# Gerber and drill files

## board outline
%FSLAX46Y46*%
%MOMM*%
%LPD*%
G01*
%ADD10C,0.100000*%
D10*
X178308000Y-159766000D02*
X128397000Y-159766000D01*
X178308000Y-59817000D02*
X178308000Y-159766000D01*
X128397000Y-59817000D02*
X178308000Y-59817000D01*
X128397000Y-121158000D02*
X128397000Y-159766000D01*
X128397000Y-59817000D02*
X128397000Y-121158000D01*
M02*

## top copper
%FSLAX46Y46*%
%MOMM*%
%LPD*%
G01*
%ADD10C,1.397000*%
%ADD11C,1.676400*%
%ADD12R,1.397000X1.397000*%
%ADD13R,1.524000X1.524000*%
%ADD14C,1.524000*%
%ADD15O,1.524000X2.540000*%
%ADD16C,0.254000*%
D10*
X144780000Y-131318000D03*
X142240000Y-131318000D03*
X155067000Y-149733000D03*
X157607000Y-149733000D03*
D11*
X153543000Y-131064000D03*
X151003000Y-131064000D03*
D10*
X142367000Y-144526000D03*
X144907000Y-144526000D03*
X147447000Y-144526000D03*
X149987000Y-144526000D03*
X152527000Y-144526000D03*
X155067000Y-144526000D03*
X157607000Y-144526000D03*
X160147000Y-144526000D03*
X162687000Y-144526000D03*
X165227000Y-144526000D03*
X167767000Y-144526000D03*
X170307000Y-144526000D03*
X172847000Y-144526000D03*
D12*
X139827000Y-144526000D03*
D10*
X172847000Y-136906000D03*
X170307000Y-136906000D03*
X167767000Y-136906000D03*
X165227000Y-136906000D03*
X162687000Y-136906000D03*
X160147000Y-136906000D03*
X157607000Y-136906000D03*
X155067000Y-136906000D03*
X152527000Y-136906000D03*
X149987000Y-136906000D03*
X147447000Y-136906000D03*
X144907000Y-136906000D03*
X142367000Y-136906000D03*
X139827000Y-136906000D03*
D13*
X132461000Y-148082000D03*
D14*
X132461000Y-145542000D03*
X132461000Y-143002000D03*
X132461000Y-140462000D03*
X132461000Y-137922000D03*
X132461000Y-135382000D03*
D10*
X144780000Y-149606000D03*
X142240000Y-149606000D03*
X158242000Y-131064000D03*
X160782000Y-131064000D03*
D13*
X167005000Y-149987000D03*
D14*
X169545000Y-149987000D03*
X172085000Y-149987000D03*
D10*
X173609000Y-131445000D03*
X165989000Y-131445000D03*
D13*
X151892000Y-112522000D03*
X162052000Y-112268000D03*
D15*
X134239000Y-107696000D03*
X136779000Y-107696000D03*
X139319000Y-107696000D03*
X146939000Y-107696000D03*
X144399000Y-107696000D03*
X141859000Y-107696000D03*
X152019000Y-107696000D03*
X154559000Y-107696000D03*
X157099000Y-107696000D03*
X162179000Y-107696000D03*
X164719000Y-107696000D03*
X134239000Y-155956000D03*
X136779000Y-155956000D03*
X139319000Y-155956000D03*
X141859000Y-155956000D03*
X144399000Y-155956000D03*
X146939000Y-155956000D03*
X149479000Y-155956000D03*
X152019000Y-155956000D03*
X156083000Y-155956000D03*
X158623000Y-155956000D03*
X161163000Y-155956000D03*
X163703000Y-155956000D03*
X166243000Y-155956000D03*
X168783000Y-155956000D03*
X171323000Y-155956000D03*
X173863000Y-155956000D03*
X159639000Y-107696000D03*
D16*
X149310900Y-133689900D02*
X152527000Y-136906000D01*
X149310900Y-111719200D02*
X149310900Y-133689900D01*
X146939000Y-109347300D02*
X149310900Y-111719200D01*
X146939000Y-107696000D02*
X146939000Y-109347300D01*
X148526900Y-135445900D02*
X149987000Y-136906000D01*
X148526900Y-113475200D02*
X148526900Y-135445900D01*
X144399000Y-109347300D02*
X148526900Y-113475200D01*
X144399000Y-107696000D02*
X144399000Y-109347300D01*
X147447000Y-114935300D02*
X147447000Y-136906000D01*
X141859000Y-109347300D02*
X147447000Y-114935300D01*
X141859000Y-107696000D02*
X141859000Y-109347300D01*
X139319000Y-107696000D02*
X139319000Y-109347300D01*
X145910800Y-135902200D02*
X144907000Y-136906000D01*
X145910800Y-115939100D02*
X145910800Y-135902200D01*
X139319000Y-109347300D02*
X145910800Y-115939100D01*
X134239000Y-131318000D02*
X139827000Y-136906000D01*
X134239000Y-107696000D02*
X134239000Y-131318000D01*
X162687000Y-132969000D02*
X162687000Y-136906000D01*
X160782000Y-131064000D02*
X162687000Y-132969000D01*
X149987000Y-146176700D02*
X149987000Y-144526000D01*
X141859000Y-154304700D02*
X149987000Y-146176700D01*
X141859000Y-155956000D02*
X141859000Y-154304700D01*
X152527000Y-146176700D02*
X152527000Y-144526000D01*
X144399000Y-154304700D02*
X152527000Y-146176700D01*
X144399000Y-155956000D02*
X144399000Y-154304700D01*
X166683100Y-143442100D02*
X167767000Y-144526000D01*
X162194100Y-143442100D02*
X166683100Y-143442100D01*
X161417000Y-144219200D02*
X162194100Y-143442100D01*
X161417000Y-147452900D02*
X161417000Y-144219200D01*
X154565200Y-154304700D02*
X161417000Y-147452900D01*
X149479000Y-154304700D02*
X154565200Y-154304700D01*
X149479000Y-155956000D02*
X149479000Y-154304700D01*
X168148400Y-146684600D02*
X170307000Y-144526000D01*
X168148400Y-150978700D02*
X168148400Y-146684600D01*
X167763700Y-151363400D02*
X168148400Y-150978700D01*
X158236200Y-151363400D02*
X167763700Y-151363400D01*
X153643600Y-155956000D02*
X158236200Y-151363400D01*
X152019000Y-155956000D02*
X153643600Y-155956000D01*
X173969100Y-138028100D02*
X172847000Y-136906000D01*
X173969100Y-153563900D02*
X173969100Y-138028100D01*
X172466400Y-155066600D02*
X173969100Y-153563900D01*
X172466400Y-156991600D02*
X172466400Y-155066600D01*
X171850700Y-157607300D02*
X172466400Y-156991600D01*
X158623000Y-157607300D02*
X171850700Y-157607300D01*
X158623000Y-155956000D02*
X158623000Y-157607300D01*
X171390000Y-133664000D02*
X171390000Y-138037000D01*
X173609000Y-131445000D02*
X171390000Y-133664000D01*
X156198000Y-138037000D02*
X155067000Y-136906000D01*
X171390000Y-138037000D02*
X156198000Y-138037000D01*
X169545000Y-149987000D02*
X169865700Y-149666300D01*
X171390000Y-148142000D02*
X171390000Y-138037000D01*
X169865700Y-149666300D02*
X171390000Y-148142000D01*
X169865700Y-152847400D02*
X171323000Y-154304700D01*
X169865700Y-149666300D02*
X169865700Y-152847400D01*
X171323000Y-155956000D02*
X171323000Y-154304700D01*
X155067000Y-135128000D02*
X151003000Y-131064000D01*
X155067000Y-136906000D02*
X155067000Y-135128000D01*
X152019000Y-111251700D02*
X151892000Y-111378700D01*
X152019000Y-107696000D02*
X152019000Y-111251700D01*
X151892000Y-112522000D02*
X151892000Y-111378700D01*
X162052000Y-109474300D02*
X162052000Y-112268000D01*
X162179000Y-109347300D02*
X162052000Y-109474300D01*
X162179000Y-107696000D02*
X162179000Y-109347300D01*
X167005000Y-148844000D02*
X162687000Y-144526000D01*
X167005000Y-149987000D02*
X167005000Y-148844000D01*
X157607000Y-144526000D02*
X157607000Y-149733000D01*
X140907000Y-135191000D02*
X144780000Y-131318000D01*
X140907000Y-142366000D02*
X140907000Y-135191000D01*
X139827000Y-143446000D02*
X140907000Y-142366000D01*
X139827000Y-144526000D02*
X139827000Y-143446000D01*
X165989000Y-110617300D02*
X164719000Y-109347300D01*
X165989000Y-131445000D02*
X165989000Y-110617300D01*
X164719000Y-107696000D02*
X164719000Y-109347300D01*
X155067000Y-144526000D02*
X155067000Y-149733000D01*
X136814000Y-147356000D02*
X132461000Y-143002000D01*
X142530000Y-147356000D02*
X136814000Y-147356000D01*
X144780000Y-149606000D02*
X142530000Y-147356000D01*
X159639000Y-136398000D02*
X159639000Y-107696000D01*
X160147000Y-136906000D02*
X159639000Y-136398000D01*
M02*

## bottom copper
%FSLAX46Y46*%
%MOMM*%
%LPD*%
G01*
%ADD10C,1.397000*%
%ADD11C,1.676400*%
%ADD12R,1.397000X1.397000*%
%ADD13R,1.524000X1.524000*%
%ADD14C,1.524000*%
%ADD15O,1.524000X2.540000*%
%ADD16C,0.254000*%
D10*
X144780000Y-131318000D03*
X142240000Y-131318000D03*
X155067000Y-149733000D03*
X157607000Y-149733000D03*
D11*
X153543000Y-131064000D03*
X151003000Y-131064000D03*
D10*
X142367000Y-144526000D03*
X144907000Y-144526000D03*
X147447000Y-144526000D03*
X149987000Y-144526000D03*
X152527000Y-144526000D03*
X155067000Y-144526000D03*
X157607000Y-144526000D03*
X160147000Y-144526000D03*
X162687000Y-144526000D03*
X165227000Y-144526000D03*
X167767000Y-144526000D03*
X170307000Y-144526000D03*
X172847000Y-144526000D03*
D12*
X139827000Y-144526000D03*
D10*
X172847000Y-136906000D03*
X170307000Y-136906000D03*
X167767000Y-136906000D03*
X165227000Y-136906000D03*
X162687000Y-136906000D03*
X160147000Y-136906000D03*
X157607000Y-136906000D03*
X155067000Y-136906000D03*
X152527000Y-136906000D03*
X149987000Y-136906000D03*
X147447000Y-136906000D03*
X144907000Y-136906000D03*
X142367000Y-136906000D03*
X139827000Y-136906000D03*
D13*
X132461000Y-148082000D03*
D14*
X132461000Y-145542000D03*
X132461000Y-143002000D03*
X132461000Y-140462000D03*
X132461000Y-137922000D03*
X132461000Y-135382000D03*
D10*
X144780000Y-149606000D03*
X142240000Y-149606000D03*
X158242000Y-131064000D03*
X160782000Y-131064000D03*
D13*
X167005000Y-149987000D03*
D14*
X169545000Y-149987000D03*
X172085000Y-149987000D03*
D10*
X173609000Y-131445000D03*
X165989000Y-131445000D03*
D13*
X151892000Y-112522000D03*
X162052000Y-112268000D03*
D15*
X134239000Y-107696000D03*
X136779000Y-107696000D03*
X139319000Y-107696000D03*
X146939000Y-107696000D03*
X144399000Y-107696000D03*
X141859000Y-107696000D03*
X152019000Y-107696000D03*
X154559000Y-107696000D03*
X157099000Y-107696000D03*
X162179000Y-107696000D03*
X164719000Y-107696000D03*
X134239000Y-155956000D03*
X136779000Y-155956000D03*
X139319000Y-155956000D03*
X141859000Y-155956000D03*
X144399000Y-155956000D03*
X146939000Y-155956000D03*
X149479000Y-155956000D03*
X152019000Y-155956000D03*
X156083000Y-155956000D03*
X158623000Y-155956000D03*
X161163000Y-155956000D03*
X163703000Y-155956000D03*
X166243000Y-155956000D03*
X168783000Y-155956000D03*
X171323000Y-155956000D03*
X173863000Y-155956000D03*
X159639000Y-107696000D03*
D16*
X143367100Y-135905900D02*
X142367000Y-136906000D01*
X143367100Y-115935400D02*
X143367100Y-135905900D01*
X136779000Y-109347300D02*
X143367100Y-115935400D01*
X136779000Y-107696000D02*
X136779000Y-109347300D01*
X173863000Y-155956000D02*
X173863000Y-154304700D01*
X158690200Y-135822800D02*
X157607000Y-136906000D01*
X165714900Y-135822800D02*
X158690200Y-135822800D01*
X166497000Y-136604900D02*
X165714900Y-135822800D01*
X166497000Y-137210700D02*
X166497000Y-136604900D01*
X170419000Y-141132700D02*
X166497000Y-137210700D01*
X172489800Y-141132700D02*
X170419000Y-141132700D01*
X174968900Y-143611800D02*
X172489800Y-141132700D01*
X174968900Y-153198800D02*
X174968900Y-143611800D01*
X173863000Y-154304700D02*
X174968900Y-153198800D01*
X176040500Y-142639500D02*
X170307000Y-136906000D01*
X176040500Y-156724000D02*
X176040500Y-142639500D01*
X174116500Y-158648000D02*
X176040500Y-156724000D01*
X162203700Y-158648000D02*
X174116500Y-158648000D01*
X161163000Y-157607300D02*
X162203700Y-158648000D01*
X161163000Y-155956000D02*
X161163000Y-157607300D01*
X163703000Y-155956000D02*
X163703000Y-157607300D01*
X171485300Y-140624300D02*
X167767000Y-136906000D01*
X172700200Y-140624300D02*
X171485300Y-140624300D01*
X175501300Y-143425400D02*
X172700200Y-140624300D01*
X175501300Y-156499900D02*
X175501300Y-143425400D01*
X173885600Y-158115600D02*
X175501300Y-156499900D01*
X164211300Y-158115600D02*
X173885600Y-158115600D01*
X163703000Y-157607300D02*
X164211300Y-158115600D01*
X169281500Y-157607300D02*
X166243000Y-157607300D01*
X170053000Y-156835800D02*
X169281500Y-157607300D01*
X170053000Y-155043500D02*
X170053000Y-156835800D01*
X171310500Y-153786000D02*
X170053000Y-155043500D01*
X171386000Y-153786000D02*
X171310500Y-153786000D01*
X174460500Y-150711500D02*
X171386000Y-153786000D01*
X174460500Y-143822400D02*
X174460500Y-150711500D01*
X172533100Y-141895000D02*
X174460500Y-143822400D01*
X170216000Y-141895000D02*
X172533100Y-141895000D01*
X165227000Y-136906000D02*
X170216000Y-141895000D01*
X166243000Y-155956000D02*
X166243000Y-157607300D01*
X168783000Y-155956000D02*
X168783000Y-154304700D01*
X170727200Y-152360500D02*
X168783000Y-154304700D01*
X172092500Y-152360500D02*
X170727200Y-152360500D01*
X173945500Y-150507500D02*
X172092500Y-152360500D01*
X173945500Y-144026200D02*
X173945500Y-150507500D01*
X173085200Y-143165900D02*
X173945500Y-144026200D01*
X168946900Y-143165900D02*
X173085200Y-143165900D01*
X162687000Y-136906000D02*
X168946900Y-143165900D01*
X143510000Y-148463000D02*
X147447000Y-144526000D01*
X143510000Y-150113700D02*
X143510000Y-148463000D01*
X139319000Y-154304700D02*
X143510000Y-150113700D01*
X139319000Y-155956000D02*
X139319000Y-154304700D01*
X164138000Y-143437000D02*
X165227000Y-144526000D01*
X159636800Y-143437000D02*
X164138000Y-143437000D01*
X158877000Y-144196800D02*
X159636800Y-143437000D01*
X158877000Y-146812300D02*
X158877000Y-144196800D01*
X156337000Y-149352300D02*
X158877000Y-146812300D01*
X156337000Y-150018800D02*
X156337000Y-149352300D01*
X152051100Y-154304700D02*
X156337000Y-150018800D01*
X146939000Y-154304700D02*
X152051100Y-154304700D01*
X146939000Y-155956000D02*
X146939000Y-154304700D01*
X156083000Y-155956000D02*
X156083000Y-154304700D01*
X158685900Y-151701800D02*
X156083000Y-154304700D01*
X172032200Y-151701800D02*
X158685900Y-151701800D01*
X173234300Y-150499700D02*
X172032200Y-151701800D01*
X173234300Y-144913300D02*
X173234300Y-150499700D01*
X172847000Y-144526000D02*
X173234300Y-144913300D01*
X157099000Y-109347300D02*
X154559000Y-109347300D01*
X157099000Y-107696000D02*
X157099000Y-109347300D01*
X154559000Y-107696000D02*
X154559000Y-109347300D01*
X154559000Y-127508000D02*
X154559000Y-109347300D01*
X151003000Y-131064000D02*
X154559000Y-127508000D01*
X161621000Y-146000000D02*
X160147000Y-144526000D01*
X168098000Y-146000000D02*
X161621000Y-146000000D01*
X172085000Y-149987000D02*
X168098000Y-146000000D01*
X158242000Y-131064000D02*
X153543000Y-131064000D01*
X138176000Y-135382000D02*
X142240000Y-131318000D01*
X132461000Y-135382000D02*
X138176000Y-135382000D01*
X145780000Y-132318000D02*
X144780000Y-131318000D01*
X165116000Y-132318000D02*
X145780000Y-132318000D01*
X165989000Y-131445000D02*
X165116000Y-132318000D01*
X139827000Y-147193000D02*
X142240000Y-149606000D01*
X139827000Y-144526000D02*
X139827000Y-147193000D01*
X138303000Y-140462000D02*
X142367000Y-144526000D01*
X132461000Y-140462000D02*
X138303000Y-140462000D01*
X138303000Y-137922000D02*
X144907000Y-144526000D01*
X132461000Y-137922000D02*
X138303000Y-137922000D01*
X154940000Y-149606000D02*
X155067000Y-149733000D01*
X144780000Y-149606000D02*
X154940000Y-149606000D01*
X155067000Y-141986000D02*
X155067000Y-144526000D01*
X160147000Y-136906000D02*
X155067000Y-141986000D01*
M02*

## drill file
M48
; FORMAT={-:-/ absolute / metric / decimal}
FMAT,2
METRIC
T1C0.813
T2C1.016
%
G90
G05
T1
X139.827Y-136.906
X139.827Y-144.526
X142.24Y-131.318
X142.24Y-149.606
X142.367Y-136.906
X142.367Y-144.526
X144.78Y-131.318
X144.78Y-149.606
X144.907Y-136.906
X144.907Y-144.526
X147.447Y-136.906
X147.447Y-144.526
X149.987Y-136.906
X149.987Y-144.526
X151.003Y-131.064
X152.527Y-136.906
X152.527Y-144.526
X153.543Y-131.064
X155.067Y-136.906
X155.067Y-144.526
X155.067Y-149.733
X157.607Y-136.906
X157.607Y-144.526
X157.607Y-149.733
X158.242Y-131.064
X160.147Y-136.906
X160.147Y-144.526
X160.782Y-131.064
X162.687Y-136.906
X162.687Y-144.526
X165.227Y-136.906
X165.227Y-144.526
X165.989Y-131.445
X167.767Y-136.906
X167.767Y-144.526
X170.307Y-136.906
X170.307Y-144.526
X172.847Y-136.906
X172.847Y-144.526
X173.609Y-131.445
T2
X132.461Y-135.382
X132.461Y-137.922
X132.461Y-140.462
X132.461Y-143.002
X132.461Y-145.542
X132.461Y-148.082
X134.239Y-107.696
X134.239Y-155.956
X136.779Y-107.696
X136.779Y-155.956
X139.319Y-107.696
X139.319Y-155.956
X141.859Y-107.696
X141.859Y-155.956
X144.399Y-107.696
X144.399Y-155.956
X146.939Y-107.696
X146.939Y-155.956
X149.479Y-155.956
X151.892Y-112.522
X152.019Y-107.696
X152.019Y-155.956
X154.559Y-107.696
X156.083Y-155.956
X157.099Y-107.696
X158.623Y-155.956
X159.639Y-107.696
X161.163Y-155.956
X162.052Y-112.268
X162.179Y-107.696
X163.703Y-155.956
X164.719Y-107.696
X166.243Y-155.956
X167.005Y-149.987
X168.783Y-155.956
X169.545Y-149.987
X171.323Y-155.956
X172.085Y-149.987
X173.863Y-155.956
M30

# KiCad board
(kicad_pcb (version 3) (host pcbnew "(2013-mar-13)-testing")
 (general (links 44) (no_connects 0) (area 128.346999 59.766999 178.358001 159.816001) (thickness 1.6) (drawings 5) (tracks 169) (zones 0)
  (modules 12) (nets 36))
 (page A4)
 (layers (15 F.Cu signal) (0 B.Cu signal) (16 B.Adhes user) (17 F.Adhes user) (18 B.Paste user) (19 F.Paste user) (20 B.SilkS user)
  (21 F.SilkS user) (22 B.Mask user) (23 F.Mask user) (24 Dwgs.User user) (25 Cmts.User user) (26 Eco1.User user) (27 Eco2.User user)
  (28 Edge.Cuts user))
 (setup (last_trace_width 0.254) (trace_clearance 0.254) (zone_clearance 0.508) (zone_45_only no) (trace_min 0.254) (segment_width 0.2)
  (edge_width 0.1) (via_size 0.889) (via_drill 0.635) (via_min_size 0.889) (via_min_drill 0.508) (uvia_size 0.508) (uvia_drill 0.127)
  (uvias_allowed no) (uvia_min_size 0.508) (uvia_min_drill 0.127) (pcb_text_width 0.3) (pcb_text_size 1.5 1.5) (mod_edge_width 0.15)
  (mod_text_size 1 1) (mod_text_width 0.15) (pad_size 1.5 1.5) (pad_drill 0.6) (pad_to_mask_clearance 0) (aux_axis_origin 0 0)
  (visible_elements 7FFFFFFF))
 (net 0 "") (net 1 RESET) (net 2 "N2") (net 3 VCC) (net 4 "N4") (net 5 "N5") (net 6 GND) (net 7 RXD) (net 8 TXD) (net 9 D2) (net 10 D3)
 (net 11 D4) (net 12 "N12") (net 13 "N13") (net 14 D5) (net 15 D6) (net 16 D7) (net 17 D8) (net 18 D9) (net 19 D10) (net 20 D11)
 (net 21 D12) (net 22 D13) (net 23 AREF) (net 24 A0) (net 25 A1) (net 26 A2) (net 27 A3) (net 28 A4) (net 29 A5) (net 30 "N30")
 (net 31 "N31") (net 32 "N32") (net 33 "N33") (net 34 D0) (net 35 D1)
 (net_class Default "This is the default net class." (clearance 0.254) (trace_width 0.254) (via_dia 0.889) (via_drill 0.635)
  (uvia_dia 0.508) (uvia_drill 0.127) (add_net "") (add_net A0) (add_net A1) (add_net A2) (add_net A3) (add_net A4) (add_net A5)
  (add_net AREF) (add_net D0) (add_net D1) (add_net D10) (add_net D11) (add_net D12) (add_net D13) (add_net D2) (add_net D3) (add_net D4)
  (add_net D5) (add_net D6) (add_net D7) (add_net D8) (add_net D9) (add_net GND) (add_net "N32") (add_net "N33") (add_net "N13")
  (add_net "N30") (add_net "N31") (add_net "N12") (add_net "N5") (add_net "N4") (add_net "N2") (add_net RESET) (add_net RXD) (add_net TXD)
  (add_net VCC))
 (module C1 (layer F.Cu) (at 143.51 131.318 180)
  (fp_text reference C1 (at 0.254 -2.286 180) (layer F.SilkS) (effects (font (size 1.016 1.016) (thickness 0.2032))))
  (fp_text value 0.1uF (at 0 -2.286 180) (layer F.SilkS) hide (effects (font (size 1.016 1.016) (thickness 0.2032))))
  (pad 1 thru_hole circle (at -1.27 0 180) (size 1.397 1.397) (drill 0.8128) (layers *.Cu *.Mask F.SilkS) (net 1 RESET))
  (pad 2 thru_hole circle (at 1.27 0 180) (size 1.397 1.397) (drill 0.8128) (layers *.Cu *.Mask F.SilkS) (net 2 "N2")))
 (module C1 (layer F.Cu) (at 156.337 149.733)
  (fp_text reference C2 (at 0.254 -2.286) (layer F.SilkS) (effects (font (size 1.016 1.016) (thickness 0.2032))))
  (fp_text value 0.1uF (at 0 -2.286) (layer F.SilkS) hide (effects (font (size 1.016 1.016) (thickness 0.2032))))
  (pad 1 thru_hole circle (at -1.27 0) (size 1.397 1.397) (drill 0.8128) (layers *.Cu *.Mask F.SilkS) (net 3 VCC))
  (pad 2 thru_hole circle (at 1.27 0) (size 1.397 1.397) (drill 0.8128) (layers *.Cu *.Mask F.SilkS) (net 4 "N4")))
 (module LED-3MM (layer F.Cu) (at 152.273 131.064 180)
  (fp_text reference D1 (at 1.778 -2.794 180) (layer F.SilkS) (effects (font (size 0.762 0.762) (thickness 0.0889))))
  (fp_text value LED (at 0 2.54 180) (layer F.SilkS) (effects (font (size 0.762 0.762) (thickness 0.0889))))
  (pad 1 thru_hole circle (at -1.27 0 180) (size 1.6764 1.6764) (drill 0.8128) (layers *.Cu *.Mask F.SilkS) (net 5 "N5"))
  (pad 2 thru_hole circle (at 1.27 0 180) (size 1.6764 1.6764) (drill 0.8128) (layers *.Cu *.Mask F.SilkS) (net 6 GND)))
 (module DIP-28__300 (layer F.Cu) (at 156.337 140.716)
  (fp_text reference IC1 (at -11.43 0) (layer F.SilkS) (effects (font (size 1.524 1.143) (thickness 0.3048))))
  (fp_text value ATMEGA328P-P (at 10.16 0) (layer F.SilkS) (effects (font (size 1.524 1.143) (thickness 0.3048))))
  (pad 2 thru_hole circle (at -13.97 3.81) (size 1.397 1.397) (drill 0.8128) (layers *.Cu *.Mask F.SilkS) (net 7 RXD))
  (pad 3 thru_hole circle (at -11.43 3.81) (size 1.397 1.397) (drill 0.8128) (layers *.Cu *.Mask F.SilkS) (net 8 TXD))
  (pad 4 thru_hole circle (at -8.89 3.81) (size 1.397 1.397) (drill 0.8128) (layers *.Cu *.Mask F.SilkS) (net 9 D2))
  (pad 5 thru_hole circle (at -6.35 3.81) (size 1.397 1.397) (drill 0.8128) (layers *.Cu *.Mask F.SilkS) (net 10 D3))
  (pad 6 thru_hole circle (at -3.81 3.81) (size 1.397 1.397) (drill 0.8128) (layers *.Cu *.Mask F.SilkS) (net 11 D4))
  (pad 7 thru_hole circle (at -1.27 3.81) (size 1.397 1.397) (drill 0.8128) (layers *.Cu *.Mask F.SilkS) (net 3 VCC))
  (pad 8 thru_hole circle (at 1.27 3.81) (size 1.397 1.397) (drill 0.8128) (layers *.Cu *.Mask F.SilkS) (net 4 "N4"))
  (pad 9 thru_hole circle (at 3.81 3.81) (size 1.397 1.397) (drill 0.8128) (layers *.Cu *.Mask F.SilkS) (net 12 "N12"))
  (pad 10 thru_hole circle (at 6.35 3.81) (size 1.397 1.397) (drill 0.8128) (layers *.Cu *.Mask F.SilkS) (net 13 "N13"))
  (pad 11 thru_hole circle (at 8.89 3.81) (size 1.397 1.397) (drill 0.8128) (layers *.Cu *.Mask F.SilkS) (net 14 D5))
  (pad 12 thru_hole circle (at 11.43 3.81) (size 1.397 1.397) (drill 0.8128) (layers *.Cu *.Mask F.SilkS) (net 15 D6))
  (pad 13 thru_hole circle (at 13.97 3.81) (size 1.397 1.397) (drill 0.8128) (layers *.Cu *.Mask F.SilkS) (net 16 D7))
  (pad 14 thru_hole circle (at 16.51 3.81) (size 1.397 1.397) (drill 0.8128) (layers *.Cu *.Mask F.SilkS) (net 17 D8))
  (pad 1 thru_hole rect (at -16.51 3.81) (size 1.397 1.397) (drill 0.8128) (layers *.Cu *.Mask F.SilkS) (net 1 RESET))
  (pad 15 thru_hole circle (at 16.51 -3.81) (size 1.397 1.397) (drill 0.8128) (layers *.Cu *.Mask F.SilkS) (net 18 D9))
  (pad 16 thru_hole circle (at 13.97 -3.81) (size 1.397 1.397) (drill 0.8128) (layers *.Cu *.Mask F.SilkS) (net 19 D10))
  (pad 17 thru_hole circle (at 11.43 -3.81) (size 1.397 1.397) (drill 0.8128) (layers *.Cu *.Mask F.SilkS) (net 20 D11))
  (pad 18 thru_hole circle (at 8.89 -3.81) (size 1.397 1.397) (drill 0.8128) (layers *.Cu *.Mask F.SilkS) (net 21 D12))
  (pad 19 thru_hole circle (at 6.35 -3.81) (size 1.397 1.397) (drill 0.8128) (layers *.Cu *.Mask F.SilkS) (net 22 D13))
  (pad 20 thru_hole circle (at 3.81 -3.81) (size 1.397 1.397) (drill 0.8128) (layers *.Cu *.Mask F.SilkS) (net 3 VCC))
  (pad 21 thru_hole circle (at 1.27 -3.81) (size 1.397 1.397) (drill 0.8128) (layers *.Cu *.Mask F.SilkS) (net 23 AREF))
  (pad 22 thru_hole circle (at -1.27 -3.81) (size 1.397 1.397) (drill 0.8128) (layers *.Cu *.Mask F.SilkS) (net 6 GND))
  (pad 23 thru_hole circle (at -3.81 -3.81) (size 1.397 1.397) (drill 0.8128) (layers *.Cu *.Mask F.SilkS) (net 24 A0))
  (pad 24 thru_hole circle (at -6.35 -3.81) (size 1.397 1.397) (drill 0.8128) (layers *.Cu *.Mask F.SilkS) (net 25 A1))
  (pad 25 thru_hole circle (at -8.89 -3.81) (size 1.397 1.397) (drill 0.8128) (layers *.Cu *.Mask F.SilkS) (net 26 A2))
  (pad 26 thru_hole circle (at -11.43 -3.81) (size 1.397 1.397) (drill 0.8128) (layers *.Cu *.Mask F.SilkS) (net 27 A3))
  (pad 27 thru_hole circle (at -13.97 -3.81) (size 1.397 1.397) (drill 0.8128) (layers *.Cu *.Mask F.SilkS) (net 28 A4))
  (pad 28 thru_hole circle (at -16.51 -3.81) (size 1.397 1.397) (drill 0.8128) (layers *.Cu *.Mask F.SilkS) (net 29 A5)))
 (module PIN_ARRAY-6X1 (layer F.Cu) (at 132.461 141.732 90)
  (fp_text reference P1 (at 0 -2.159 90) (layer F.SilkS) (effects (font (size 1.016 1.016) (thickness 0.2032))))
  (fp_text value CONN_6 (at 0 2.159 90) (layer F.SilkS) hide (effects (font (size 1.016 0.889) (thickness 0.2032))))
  (pad 1 thru_hole rect (at -6.35 0 90) (size 1.524 1.524) (drill 1.016) (layers *.Cu *.Mask F.SilkS) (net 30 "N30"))
  (pad 2 thru_hole circle (at -3.81 0 90) (size 1.524 1.524) (drill 1.016) (layers *.Cu *.Mask F.SilkS) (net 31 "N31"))
  (pad 3 thru_hole circle (at -1.27 0 90) (size 1.524 1.524) (drill 1.016) (layers *.Cu *.Mask F.SilkS) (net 3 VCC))
  (pad 4 thru_hole circle (at 1.27 0 90) (size 1.524 1.524) (drill 1.016) (layers *.Cu *.Mask F.SilkS) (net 7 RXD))
  (pad 5 thru_hole circle (at 3.81 0 90) (size 1.524 1.524) (drill 1.016) (layers *.Cu *.Mask F.SilkS) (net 8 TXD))
  (pad 6 thru_hole circle (at 6.35 0 90) (size 1.524 1.524) (drill 1.016) (layers *.Cu *.Mask F.SilkS) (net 2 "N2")))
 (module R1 (layer F.Cu) (at 143.51 149.606 180) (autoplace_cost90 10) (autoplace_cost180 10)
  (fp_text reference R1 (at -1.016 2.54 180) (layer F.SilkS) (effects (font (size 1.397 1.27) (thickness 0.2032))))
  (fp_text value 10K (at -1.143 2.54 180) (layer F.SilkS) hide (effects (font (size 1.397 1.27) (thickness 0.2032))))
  (pad 1 thru_hole circle (at -1.27 0 180) (size 1.397 1.397) (drill 0.8128) (layers *.Cu *.Mask F.SilkS) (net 3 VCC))
  (pad 2 thru_hole circle (at 1.27 0 180) (size 1.397 1.397) (drill 0.8128) (layers *.Cu *.Mask F.SilkS) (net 1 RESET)))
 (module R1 (layer F.Cu) (at 159.512 131.064) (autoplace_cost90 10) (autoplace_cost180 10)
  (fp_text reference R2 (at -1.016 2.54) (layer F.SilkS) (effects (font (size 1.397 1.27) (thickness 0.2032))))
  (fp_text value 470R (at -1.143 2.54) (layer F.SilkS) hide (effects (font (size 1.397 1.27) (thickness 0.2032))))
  (pad 1 thru_hole circle (at -1.27 0) (size 1.397 1.397) (drill 0.8128) (layers *.Cu *.Mask F.SilkS) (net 5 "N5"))
  (pad 2 thru_hole circle (at 1.27 0) (size 1.397 1.397) (drill 0.8128) (layers *.Cu *.Mask F.SilkS) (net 22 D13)))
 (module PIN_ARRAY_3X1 (layer F.Cu) (at 169.545 149.987)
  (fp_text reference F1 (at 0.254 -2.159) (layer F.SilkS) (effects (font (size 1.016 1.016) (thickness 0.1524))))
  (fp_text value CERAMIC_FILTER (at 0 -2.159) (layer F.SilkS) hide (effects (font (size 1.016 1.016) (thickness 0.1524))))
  (pad 1 thru_hole rect (at -2.54 0) (size 1.524 1.524) (drill 1.016) (layers *.Cu *.Mask F.SilkS) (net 13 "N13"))
  (pad 2 thru_hole circle (at 0 0) (size 1.524 1.524) (drill 1.016) (layers *.Cu *.Mask F.SilkS) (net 6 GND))
  (pad 3 thru_hole circle (at 2.54 0) (size 1.524 1.524) (drill 1.016) (layers *.Cu *.Mask F.SilkS) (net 12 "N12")))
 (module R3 (layer F.Cu) (at 169.799 131.445 180) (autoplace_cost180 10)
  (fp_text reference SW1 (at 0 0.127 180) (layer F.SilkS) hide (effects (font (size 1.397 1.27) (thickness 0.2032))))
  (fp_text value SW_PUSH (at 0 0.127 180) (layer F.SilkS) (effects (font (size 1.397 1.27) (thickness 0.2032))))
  (pad 1 thru_hole circle (at -3.81 0 180) (size 1.397 1.397) (drill 0.8128) (layers *.Cu *.Mask F.SilkS) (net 6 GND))
  (pad 2 thru_hole circle (at 3.81 0 180) (size 1.397 1.397) (drill 0.8128) (layers *.Cu *.Mask F.SilkS) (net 1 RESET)))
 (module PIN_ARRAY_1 (layer F.Cu) (at 151.892 112.522)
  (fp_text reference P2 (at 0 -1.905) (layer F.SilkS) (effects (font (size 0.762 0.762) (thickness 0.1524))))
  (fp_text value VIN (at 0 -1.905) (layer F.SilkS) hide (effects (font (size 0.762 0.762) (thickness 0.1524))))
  (pad 1 thru_hole rect (at 0 0) (size 1.524 1.524) (drill 1.016) (layers *.Cu *.Mask F.SilkS) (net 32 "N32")))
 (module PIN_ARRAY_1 (layer F.Cu) (at 162.052 112.268)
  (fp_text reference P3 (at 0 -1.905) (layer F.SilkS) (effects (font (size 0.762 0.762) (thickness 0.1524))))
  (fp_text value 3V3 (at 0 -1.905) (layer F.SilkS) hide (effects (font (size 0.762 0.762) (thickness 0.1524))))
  (pad 1 thru_hole rect (at 0 0) (size 1.524 1.524) (drill 1.016) (layers *.Cu *.Mask F.SilkS) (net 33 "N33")))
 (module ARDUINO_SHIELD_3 (layer F.Cu) (at 174.879 106.426 180)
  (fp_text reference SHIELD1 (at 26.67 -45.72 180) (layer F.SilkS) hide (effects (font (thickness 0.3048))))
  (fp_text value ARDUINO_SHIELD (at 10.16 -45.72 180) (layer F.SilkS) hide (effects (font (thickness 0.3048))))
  (pad AD5 thru_hole oval (at 40.64 -1.27 270) (size 2.54 1.524) (drill 1.016) (layers *.Cu *.Mask F.SilkS) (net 29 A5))
  (pad AD4 thru_hole oval (at 38.1 -1.27 270) (size 2.54 1.524) (drill 1.016) (layers *.Cu *.Mask F.SilkS) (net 28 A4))
  (pad AD3 thru_hole oval (at 35.56 -1.27 270) (size 2.54 1.524) (drill 1.016) (layers *.Cu *.Mask F.SilkS) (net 27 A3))
  (pad AD0 thru_hole oval (at 27.94 -1.27 270) (size 2.54 1.524) (drill 1.016) (layers *.Cu *.Mask F.SilkS) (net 24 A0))
  (pad AD1 thru_hole oval (at 30.48 -1.27 270) (size 2.54 1.524) (drill 1.016) (layers *.Cu *.Mask F.SilkS) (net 25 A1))
  (pad AD2 thru_hole oval (at 33.02 -1.27 270) (size 2.54 1.524) (drill 1.016) (layers *.Cu *.Mask F.SilkS) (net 26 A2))
  (pad V_IN thru_hole oval (at 22.86 -1.27 270) (size 2.54 1.524) (drill 1.016) (layers *.Cu *.Mask F.SilkS) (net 32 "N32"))
  (pad GND2 thru_hole oval (at 20.32 -1.27 270) (size 2.54 1.524) (drill 1.016) (layers *.Cu *.Mask F.SilkS) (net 6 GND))
  (pad GND1 thru_hole oval (at 17.78 -1.27 270) (size 2.54 1.524) (drill 1.016) (layers *.Cu *.Mask F.SilkS) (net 6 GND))
  (pad 3V3 thru_hole oval (at 12.7 -1.27 270) (size 2.54 1.524) (drill 1.016) (layers *.Cu *.Mask F.SilkS) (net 33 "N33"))
  (pad RST thru_hole oval (at 10.16 -1.27 270) (size 2.54 1.524) (drill 1.016) (layers *.Cu *.Mask F.SilkS) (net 1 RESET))
  (pad 0 thru_hole oval (at 40.64 -49.53 270) (size 2.54 1.524) (drill 1.016) (layers *.Cu *.Mask F.SilkS) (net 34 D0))
  (pad 1 thru_hole oval (at 38.1 -49.53 270) (size 2.54 1.524) (drill 1.016) (layers *.Cu *.Mask F.SilkS) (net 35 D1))
  (pad 2 thru_hole oval (at 35.56 -49.53 270) (size 2.54 1.524) (drill 1.016) (layers *.Cu *.Mask F.SilkS) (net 9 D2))
  (pad 3 thru_hole oval (at 33.02 -49.53 270) (size 2.54 1.524) (drill 1.016) (layers *.Cu *.Mask F.SilkS) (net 10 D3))
  (pad 4 thru_hole oval (at 30.48 -49.53 270) (size 2.54 1.524) (drill 1.016) (layers *.Cu *.Mask F.SilkS) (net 11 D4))
  (pad 5 thru_hole oval (at 27.94 -49.53 270) (size 2.54 1.524) (drill 1.016) (layers *.Cu *.Mask F.SilkS) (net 14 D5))
  (pad 6 thru_hole oval (at 25.4 -49.53 270) (size 2.54 1.524) (drill 1.016) (layers *.Cu *.Mask F.SilkS) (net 15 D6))
  (pad 7 thru_hole oval (at 22.86 -49.53 270) (size 2.54 1.524) (drill 1.016) (layers *.Cu *.Mask F.SilkS) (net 16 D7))
  (pad 8 thru_hole oval (at 18.796 -49.53 270) (size 2.54 1.524) (drill 1.016) (layers *.Cu *.Mask F.SilkS) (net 17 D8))
  (pad 9 thru_hole oval (at 16.256 -49.53 270) (size 2.54 1.524) (drill 1.016) (layers *.Cu *.Mask F.SilkS) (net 18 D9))
  (pad 10 thru_hole oval (at 13.716 -49.53 270) (size 2.54 1.524) (drill 1.016) (layers *.Cu *.Mask F.SilkS) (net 19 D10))
  (pad 11 thru_hole oval (at 11.176 -49.53 270) (size 2.54 1.524) (drill 1.016) (layers *.Cu *.Mask F.SilkS) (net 20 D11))
  (pad 12 thru_hole oval (at 8.636 -49.53 270) (size 2.54 1.524) (drill 1.016) (layers *.Cu *.Mask F.SilkS) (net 21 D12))
  (pad 13 thru_hole oval (at 6.096 -49.53 270) (size 2.54 1.524) (drill 1.016) (layers *.Cu *.Mask F.SilkS) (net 22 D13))
  (pad GND3 thru_hole oval (at 3.556 -49.53 270) (size 2.54 1.524) (drill 1.016) (layers *.Cu *.Mask F.SilkS) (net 6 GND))
  (pad AREF thru_hole oval (at 1.016 -49.53 270) (size 2.54 1.524) (drill 1.016) (layers *.Cu *.Mask F.SilkS) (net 23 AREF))
  (pad 5V thru_hole oval (at 15.24 -1.27 270) (size 2.54 1.524) (drill 1.016) (layers *.Cu *.Mask F.SilkS) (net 3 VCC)))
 (gr_line (start 178.308 159.766) (end 128.397 159.766) (angle 90) (layer Edge.Cuts) (width 0.1))
 (gr_line (start 178.308 59.817) (end 178.308 159.766) (angle 90) (layer Edge.Cuts) (width 0.1))
 (gr_line (start 128.397 59.817) (end 178.308 59.817) (angle 90) (layer Edge.Cuts) (width 0.1))
 (gr_line (start 128.397 121.158) (end 128.397 159.766) (angle 90) (layer Edge.Cuts) (width 0.1))
 (gr_line (start 128.397 59.817) (end 128.397 121.158) (angle 90) (layer Edge.Cuts) (width 0.1))
 (segment (start 149.3109 133.6899) (end 152.527 136.906) (width 0.254) (layer F.Cu) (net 24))
 (segment (start 149.3109 111.7192) (end 149.3109 133.6899) (width 0.254) (layer F.Cu) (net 24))
 (segment (start 146.939 109.3473) (end 149.3109 111.7192) (width 0.254) (layer F.Cu) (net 24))
 (segment (start 146.939 107.696) (end 146.939 109.3473) (width 0.254) (layer F.Cu) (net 24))
 (segment (start 148.5269 135.4459) (end 149.987 136.906) (width 0.254) (layer F.Cu) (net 25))
 (segment (start 148.5269 113.4752) (end 148.5269 135.4459) (width 0.254) (layer F.Cu) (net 25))
 (segment (start 144.399 109.3473) (end 148.5269 113.4752) (width 0.254) (layer F.Cu) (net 25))
 (segment (start 144.399 107.696) (end 144.399 109.3473) (width 0.254) (layer F.Cu) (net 25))
 (segment (start 147.447 114.9353) (end 147.447 136.906) (width 0.254) (layer F.Cu) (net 26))
 (segment (start 141.859 109.3473) (end 147.447 114.9353) (width 0.254) (layer F.Cu) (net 26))
 (segment (start 141.859 107.696) (end 141.859 109.3473) (width 0.254) (layer F.Cu) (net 26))
 (segment (start 139.319 107.696) (end 139.319 109.3473) (width 0.254) (layer F.Cu) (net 27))
 (segment (start 145.9108 135.9022) (end 144.907 136.906) (width 0.254) (layer F.Cu) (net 27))
 (segment (start 145.9108 115.9391) (end 145.9108 135.9022) (width 0.254) (layer F.Cu) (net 27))
 (segment (start 139.319 109.3473) (end 145.9108 115.9391) (width 0.254) (layer F.Cu) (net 27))
 (segment (start 143.3671 135.9059) (end 142.367 136.906) (width 0.254) (layer B.Cu) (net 28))
 (segment (start 143.3671 115.9354) (end 143.3671 135.9059) (width 0.254) (layer B.Cu) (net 28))
 (segment (start 136.779 109.3473) (end 143.3671 115.9354) (width 0.254) (layer B.Cu) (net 28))
 (segment (start 136.779 107.696) (end 136.779 109.3473) (width 0.254) (layer B.Cu) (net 28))
 (segment (start 134.239 131.318) (end 139.827 136.906) (width 0.254) (layer F.Cu) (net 29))
 (segment (start 134.239 107.696) (end 134.239 131.318) (width 0.254) (layer F.Cu) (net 29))
 (segment (start 173.863 155.956) (end 173.863 154.3047) (width 0.254) (layer B.Cu) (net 23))
 (segment (start 158.6902 135.8228) (end 157.607 136.906) (width 0.254) (layer B.Cu) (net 23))
 (segment (start 165.7149 135.8228) (end 158.6902 135.8228) (width 0.254) (layer B.Cu) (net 23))
 (segment (start 166.497 136.6049) (end 165.7149 135.8228) (width 0.254) (layer B.Cu) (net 23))
 (segment (start 166.497 137.2107) (end 166.497 136.6049) (width 0.254) (layer B.Cu) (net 23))
 (segment (start 170.419 141.1327) (end 166.497 137.2107) (width 0.254) (layer B.Cu) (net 23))
 (segment (start 172.4898 141.1327) (end 170.419 141.1327) (width 0.254) (layer B.Cu) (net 23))
 (segment (start 174.9689 143.6118) (end 172.4898 141.1327) (width 0.254) (layer B.Cu) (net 23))
 (segment (start 174.9689 153.1988) (end 174.9689 143.6118) (width 0.254) (layer B.Cu) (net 23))
 (segment (start 173.863 154.3047) (end 174.9689 153.1988) (width 0.254) (layer B.Cu) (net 23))
 (segment (start 176.0405 142.6395) (end 170.307 136.906) (width 0.254) (layer B.Cu) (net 19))
 (segment (start 176.0405 156.724) (end 176.0405 142.6395) (width 0.254) (layer B.Cu) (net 19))
 (segment (start 174.1165 158.648) (end 176.0405 156.724) (width 0.254) (layer B.Cu) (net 19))
 (segment (start 162.2037 158.648) (end 174.1165 158.648) (width 0.254) (layer B.Cu) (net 19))
 (segment (start 161.163 157.6073) (end 162.2037 158.648) (width 0.254) (layer B.Cu) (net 19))
 (segment (start 161.163 155.956) (end 161.163 157.6073) (width 0.254) (layer B.Cu) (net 19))
 (segment (start 163.703 155.956) (end 163.703 157.6073) (width 0.254) (layer B.Cu) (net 20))
 (segment (start 171.4853 140.6243) (end 167.767 136.906) (width 0.254) (layer B.Cu) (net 20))
 (segment (start 172.7002 140.6243) (end 171.4853 140.6243) (width 0.254) (layer B.Cu) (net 20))
 (segment (start 175.5013 143.4254) (end 172.7002 140.6243) (width 0.254) (layer B.Cu) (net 20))
 (segment (start 175.5013 156.4999) (end 175.5013 143.4254) (width 0.254) (layer B.Cu) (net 20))
 (segment (start 173.8856 158.1156) (end 175.5013 156.4999) (width 0.254) (layer B.Cu) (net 20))
 (segment (start 164.2113 158.1156) (end 173.8856 158.1156) (width 0.254) (layer B.Cu) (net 20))
 (segment (start 163.703 157.6073) (end 164.2113 158.1156) (width 0.254) (layer B.Cu) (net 20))
 (segment (start 169.2815 157.6073) (end 166.243 157.6073) (width 0.254) (layer B.Cu) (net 21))
 (segment (start 170.053 156.8358) (end 169.2815 157.6073) (width 0.254) (layer B.Cu) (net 21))
 (segment (start 170.053 155.0435) (end 170.053 156.8358) (width 0.254) (layer B.Cu) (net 21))
 (segment (start 171.3105 153.786) (end 170.053 155.0435) (width 0.254) (layer B.Cu) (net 21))
 (segment (start 171.386 153.786) (end 171.3105 153.786) (width 0.254) (layer B.Cu) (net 21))
 (segment (start 174.4605 150.7115) (end 171.386 153.786) (width 0.254) (layer B.Cu) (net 21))
 (segment (start 174.4605 143.8224) (end 174.4605 150.7115) (width 0.254) (layer B.Cu) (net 21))
 (segment (start 172.5331 141.895) (end 174.4605 143.8224) (width 0.254) (layer B.Cu) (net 21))
 (segment (start 170.216 141.895) (end 172.5331 141.895) (width 0.254) (layer B.Cu) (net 21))
 (segment (start 165.227 136.906) (end 170.216 141.895) (width 0.254) (layer B.Cu) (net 21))
 (segment (start 166.243 155.956) (end 166.243 157.6073) (width 0.254) (layer B.Cu) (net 21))
 (segment (start 162.687 132.969) (end 162.687 136.906) (width 0.254) (layer F.Cu) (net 22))
 (segment (start 160.782 131.064) (end 162.687 132.969) (width 0.254) (layer F.Cu) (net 22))
 (segment (start 168.783 155.956) (end 168.783 154.3047) (width 0.254) (layer B.Cu) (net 22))
 (segment (start 170.7272 152.3605) (end 168.783 154.3047) (width 0.254) (layer B.Cu) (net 22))
 (segment (start 172.0925 152.3605) (end 170.7272 152.3605) (width 0.254) (layer B.Cu) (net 22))
 (segment (start 173.9455 150.5075) (end 172.0925 152.3605) (width 0.254) (layer B.Cu) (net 22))
 (segment (start 173.9455 144.0262) (end 173.9455 150.5075) (width 0.254) (layer B.Cu) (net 22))
 (segment (start 173.0852 143.1659) (end 173.9455 144.0262) (width 0.254) (layer B.Cu) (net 22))
 (segment (start 168.9469 143.1659) (end 173.0852 143.1659) (width 0.254) (layer B.Cu) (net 22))
 (segment (start 162.687 136.906) (end 168.9469 143.1659) (width 0.254) (layer B.Cu) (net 22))
 (segment (start 143.51 148.463) (end 147.447 144.526) (width 0.254) (layer B.Cu) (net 9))
 (segment (start 143.51 150.1137) (end 143.51 148.463) (width 0.254) (layer B.Cu) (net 9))
 (segment (start 139.319 154.3047) (end 143.51 150.1137) (width 0.254) (layer B.Cu) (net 9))
 (segment (start 139.319 155.956) (end 139.319 154.3047) (width 0.254) (layer B.Cu) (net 9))
 (segment (start 149.987 146.1767) (end 149.987 144.526) (width 0.254) (layer F.Cu) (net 10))
 (segment (start 141.859 154.3047) (end 149.987 146.1767) (width 0.254) (layer F.Cu) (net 10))
 (segment (start 141.859 155.956) (end 141.859 154.3047) (width 0.254) (layer F.Cu) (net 10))
 (segment (start 152.527 146.1767) (end 152.527 144.526) (width 0.254) (layer F.Cu) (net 11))
 (segment (start 144.399 154.3047) (end 152.527 146.1767) (width 0.254) (layer F.Cu) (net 11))
 (segment (start 144.399 155.956) (end 144.399 154.3047) (width 0.254) (layer F.Cu) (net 11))
 (segment (start 164.138 143.437) (end 165.227 144.526) (width 0.254) (layer B.Cu) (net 14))
 (segment (start 159.6368 143.437) (end 164.138 143.437) (width 0.254) (layer B.Cu) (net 14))
 (segment (start 158.877 144.1968) (end 159.6368 143.437) (width 0.254) (layer B.Cu) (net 14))
 (segment (start 158.877 146.8123) (end 158.877 144.1968) (width 0.254) (layer B.Cu) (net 14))
 (segment (start 156.337 149.3523) (end 158.877 146.8123) (width 0.254) (layer B.Cu) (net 14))
 (segment (start 156.337 150.0188) (end 156.337 149.3523) (width 0.254) (layer B.Cu) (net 14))
 (segment (start 152.0511 154.3047) (end 156.337 150.0188) (width 0.254) (layer B.Cu) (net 14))
 (segment (start 146.939 154.3047) (end 152.0511 154.3047) (width 0.254) (layer B.Cu) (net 14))
 (segment (start 146.939 155.956) (end 146.939 154.3047) (width 0.254) (layer B.Cu) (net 14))
 (segment (start 166.6831 143.4421) (end 167.767 144.526) (width 0.254) (layer F.Cu) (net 15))
 (segment (start 162.1941 143.4421) (end 166.6831 143.4421) (width 0.254) (layer F.Cu) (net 15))
 (segment (start 161.417 144.2192) (end 162.1941 143.4421) (width 0.254) (layer F.Cu) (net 15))
 (segment (start 161.417 147.4529) (end 161.417 144.2192) (width 0.254) (layer F.Cu) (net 15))
 (segment (start 154.5652 154.3047) (end 161.417 147.4529) (width 0.254) (layer F.Cu) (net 15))
 (segment (start 149.479 154.3047) (end 154.5652 154.3047) (width 0.254) (layer F.Cu) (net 15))
 (segment (start 149.479 155.956) (end 149.479 154.3047) (width 0.254) (layer F.Cu) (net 15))
 (segment (start 168.1484 146.6846) (end 170.307 144.526) (width 0.254) (layer F.Cu) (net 16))
 (segment (start 168.1484 150.9787) (end 168.1484 146.6846) (width 0.254) (layer F.Cu) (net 16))
 (segment (start 167.7637 151.3634) (end 168.1484 150.9787) (width 0.254) (layer F.Cu) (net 16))
 (segment (start 158.2362 151.3634) (end 167.7637 151.3634) (width 0.254) (layer F.Cu) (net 16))
 (segment (start 153.6436 155.956) (end 158.2362 151.3634) (width 0.254) (layer F.Cu) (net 16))
 (segment (start 152.019 155.956) (end 153.6436 155.956) (width 0.254) (layer F.Cu) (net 16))
 (segment (start 156.083 155.956) (end 156.083 154.3047) (width 0.254) (layer B.Cu) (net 17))
 (segment (start 158.6859 151.7018) (end 156.083 154.3047) (width 0.254) (layer B.Cu) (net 17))
 (segment (start 172.0322 151.7018) (end 158.6859 151.7018) (width 0.254) (layer B.Cu) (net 17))
 (segment (start 173.2343 150.4997) (end 172.0322 151.7018) (width 0.254) (layer B.Cu) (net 17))
 (segment (start 173.2343 144.9133) (end 173.2343 150.4997) (width 0.254) (layer B.Cu) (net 17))
 (segment (start 172.847 144.526) (end 173.2343 144.9133) (width 0.254) (layer B.Cu) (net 17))
 (segment (start 173.9691 138.0281) (end 172.847 136.906) (width 0.254) (layer F.Cu) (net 18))
 (segment (start 173.9691 153.5639) (end 173.9691 138.0281) (width 0.254) (layer F.Cu) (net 18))
 (segment (start 172.4664 155.0666) (end 173.9691 153.5639) (width 0.254) (layer F.Cu) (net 18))
 (segment (start 172.4664 156.9916) (end 172.4664 155.0666) (width 0.254) (layer F.Cu) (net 18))
 (segment (start 171.8507 157.6073) (end 172.4664 156.9916) (width 0.254) (layer F.Cu) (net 18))
 (segment (start 158.623 157.6073) (end 171.8507 157.6073) (width 0.254) (layer F.Cu) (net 18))
 (segment (start 158.623 155.956) (end 158.623 157.6073) (width 0.254) (layer F.Cu) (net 18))
 (segment (start 171.39 133.664) (end 171.39 138.037) (width 0.254) (layer F.Cu) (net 6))
 (segment (start 173.609 131.445) (end 171.39 133.664) (width 0.254) (layer F.Cu) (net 6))
 (segment (start 156.198 138.037) (end 155.067 136.906) (width 0.254) (layer F.Cu) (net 6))
 (segment (start 171.39 138.037) (end 156.198 138.037) (width 0.254) (layer F.Cu) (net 6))
 (segment (start 169.545 149.987) (end 169.8657 149.6663) (width 0.254) (layer F.Cu) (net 6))
 (segment (start 171.39 148.142) (end 171.39 138.037) (width 0.254) (layer F.Cu) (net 6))
 (segment (start 169.8657 149.6663) (end 171.39 148.142) (width 0.254) (layer F.Cu) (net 6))
 (segment (start 169.8657 152.8474) (end 171.323 154.3047) (width 0.254) (layer F.Cu) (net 6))
 (segment (start 169.8657 149.6663) (end 169.8657 152.8474) (width 0.254) (layer F.Cu) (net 6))
 (segment (start 171.323 155.956) (end 171.323 154.3047) (width 0.254) (layer F.Cu) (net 6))
 (segment (start 155.067 135.128) (end 151.003 131.064) (width 0.254) (layer F.Cu) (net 6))
 (segment (start 155.067 136.906) (end 155.067 135.128) (width 0.254) (layer F.Cu) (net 6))
 (segment (start 157.099 109.3473) (end 154.559 109.3473) (width 0.254) (layer B.Cu) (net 6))
 (segment (start 157.099 107.696) (end 157.099 109.3473) (width 0.254) (layer B.Cu) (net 6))
 (segment (start 154.559 107.696) (end 154.559 109.3473) (width 0.254) (layer B.Cu) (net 6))
 (segment (start 154.559 127.508) (end 154.559 109.3473) (width 0.254) (layer B.Cu) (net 6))
 (segment (start 151.003 131.064) (end 154.559 127.508) (width 0.254) (layer B.Cu) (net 6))
 (segment (start 152.019 111.2517) (end 151.892 111.3787) (width 0.254) (layer F.Cu) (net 32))
 (segment (start 152.019 107.696) (end 152.019 111.2517) (width 0.254) (layer F.Cu) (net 32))
 (segment (start 151.892 112.522) (end 151.892 111.3787) (width 0.254) (layer F.Cu) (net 32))
 (segment (start 162.052 109.4743) (end 162.052 112.268) (width 0.254) (layer F.Cu) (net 33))
 (segment (start 162.179 109.3473) (end 162.052 109.4743) (width 0.254) (layer F.Cu) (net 33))
 (segment (start 162.179 107.696) (end 162.179 109.3473) (width 0.254) (layer F.Cu) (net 33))
 (segment (start 167.005 148.844) (end 162.687 144.526) (width 0.254) (layer F.Cu) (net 13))
 (segment (start 167.005 149.987) (end 167.005 148.844) (width 0.254) (layer F.Cu) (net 13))
 (segment (start 161.621 146) (end 160.147 144.526) (width 0.254) (layer B.Cu) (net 12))
 (segment (start 168.098 146) (end 161.621 146) (width 0.254) (layer B.Cu) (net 12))
 (segment (start 172.085 149.987) (end 168.098 146) (width 0.254) (layer B.Cu) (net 12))
 (segment (start 158.242 131.064) (end 153.543 131.064) (width 0.254) (layer B.Cu) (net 5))
 (segment (start 157.607 144.526) (end 157.607 149.733) (width 0.254) (layer F.Cu) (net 4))
 (segment (start 138.176 135.382) (end 142.24 131.318) (width 0.254) (layer B.Cu) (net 2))
 (segment (start 132.461 135.382) (end 138.176 135.382) (width 0.254) (layer B.Cu) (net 2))
 (segment (start 145.78 132.318) (end 144.78 131.318) (width 0.254) (layer B.Cu) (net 1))
 (segment (start 165.116 132.318) (end 145.78 132.318) (width 0.254) (layer B.Cu) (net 1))
 (segment (start 165.989 131.445) (end 165.116 132.318) (width 0.254) (layer B.Cu) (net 1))
 (segment (start 140.907 135.191) (end 144.78 131.318) (width 0.254) (layer F.Cu) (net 1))
 (segment (start 140.907 142.366) (end 140.907 135.191) (width 0.254) (layer F.Cu) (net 1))
 (segment (start 139.827 143.446) (end 140.907 142.366) (width 0.254) (layer F.Cu) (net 1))
 (segment (start 139.827 144.526) (end 139.827 143.446) (width 0.254) (layer F.Cu) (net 1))
 (segment (start 139.827 147.193) (end 142.24 149.606) (width 0.254) (layer B.Cu) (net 1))
 (segment (start 139.827 144.526) (end 139.827 147.193) (width 0.254) (layer B.Cu) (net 1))
 (segment (start 165.989 110.6173) (end 164.719 109.3473) (width 0.254) (layer F.Cu) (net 1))
 (segment (start 165.989 131.445) (end 165.989 110.6173) (width 0.254) (layer F.Cu) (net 1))
 (segment (start 164.719 107.696) (end 164.719 109.3473) (width 0.254) (layer F.Cu) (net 1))
 (segment (start 138.303 140.462) (end 142.367 144.526) (width 0.254) (layer B.Cu) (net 7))
 (segment (start 132.461 140.462) (end 138.303 140.462) (width 0.254) (layer B.Cu) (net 7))
 (segment (start 138.303 137.922) (end 144.907 144.526) (width 0.254) (layer B.Cu) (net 8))
 (segment (start 132.461 137.922) (end 138.303 137.922) (width 0.254) (layer B.Cu) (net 8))
 (segment (start 154.94 149.606) (end 155.067 149.733) (width 0.254) (layer B.Cu) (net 3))
 (segment (start 144.78 149.606) (end 154.94 149.606) (width 0.254) (layer B.Cu) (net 3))
 (segment (start 155.067 141.986) (end 155.067 144.526) (width 0.254) (layer B.Cu) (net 3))
 (segment (start 160.147 136.906) (end 155.067 141.986) (width 0.254) (layer B.Cu) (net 3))
 (segment (start 155.067 144.526) (end 155.067 149.733) (width 0.254) (layer F.Cu) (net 3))
 (segment (start 136.814 147.356) (end 132.461 143.002) (width 0.254) (layer F.Cu) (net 3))
 (segment (start 142.53 147.356) (end 136.814 147.356) (width 0.254) (layer F.Cu) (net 3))
 (segment (start 144.78 149.606) (end 142.53 147.356) (width 0.254) (layer F.Cu) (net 3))
 (segment (start 159.639 136.398) (end 159.639 107.696) (width 0.254) (layer F.Cu) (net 3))
 (segment (start 160.147 136.906) (end 159.639 136.398) (width 0.254) (layer F.Cu) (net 3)))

